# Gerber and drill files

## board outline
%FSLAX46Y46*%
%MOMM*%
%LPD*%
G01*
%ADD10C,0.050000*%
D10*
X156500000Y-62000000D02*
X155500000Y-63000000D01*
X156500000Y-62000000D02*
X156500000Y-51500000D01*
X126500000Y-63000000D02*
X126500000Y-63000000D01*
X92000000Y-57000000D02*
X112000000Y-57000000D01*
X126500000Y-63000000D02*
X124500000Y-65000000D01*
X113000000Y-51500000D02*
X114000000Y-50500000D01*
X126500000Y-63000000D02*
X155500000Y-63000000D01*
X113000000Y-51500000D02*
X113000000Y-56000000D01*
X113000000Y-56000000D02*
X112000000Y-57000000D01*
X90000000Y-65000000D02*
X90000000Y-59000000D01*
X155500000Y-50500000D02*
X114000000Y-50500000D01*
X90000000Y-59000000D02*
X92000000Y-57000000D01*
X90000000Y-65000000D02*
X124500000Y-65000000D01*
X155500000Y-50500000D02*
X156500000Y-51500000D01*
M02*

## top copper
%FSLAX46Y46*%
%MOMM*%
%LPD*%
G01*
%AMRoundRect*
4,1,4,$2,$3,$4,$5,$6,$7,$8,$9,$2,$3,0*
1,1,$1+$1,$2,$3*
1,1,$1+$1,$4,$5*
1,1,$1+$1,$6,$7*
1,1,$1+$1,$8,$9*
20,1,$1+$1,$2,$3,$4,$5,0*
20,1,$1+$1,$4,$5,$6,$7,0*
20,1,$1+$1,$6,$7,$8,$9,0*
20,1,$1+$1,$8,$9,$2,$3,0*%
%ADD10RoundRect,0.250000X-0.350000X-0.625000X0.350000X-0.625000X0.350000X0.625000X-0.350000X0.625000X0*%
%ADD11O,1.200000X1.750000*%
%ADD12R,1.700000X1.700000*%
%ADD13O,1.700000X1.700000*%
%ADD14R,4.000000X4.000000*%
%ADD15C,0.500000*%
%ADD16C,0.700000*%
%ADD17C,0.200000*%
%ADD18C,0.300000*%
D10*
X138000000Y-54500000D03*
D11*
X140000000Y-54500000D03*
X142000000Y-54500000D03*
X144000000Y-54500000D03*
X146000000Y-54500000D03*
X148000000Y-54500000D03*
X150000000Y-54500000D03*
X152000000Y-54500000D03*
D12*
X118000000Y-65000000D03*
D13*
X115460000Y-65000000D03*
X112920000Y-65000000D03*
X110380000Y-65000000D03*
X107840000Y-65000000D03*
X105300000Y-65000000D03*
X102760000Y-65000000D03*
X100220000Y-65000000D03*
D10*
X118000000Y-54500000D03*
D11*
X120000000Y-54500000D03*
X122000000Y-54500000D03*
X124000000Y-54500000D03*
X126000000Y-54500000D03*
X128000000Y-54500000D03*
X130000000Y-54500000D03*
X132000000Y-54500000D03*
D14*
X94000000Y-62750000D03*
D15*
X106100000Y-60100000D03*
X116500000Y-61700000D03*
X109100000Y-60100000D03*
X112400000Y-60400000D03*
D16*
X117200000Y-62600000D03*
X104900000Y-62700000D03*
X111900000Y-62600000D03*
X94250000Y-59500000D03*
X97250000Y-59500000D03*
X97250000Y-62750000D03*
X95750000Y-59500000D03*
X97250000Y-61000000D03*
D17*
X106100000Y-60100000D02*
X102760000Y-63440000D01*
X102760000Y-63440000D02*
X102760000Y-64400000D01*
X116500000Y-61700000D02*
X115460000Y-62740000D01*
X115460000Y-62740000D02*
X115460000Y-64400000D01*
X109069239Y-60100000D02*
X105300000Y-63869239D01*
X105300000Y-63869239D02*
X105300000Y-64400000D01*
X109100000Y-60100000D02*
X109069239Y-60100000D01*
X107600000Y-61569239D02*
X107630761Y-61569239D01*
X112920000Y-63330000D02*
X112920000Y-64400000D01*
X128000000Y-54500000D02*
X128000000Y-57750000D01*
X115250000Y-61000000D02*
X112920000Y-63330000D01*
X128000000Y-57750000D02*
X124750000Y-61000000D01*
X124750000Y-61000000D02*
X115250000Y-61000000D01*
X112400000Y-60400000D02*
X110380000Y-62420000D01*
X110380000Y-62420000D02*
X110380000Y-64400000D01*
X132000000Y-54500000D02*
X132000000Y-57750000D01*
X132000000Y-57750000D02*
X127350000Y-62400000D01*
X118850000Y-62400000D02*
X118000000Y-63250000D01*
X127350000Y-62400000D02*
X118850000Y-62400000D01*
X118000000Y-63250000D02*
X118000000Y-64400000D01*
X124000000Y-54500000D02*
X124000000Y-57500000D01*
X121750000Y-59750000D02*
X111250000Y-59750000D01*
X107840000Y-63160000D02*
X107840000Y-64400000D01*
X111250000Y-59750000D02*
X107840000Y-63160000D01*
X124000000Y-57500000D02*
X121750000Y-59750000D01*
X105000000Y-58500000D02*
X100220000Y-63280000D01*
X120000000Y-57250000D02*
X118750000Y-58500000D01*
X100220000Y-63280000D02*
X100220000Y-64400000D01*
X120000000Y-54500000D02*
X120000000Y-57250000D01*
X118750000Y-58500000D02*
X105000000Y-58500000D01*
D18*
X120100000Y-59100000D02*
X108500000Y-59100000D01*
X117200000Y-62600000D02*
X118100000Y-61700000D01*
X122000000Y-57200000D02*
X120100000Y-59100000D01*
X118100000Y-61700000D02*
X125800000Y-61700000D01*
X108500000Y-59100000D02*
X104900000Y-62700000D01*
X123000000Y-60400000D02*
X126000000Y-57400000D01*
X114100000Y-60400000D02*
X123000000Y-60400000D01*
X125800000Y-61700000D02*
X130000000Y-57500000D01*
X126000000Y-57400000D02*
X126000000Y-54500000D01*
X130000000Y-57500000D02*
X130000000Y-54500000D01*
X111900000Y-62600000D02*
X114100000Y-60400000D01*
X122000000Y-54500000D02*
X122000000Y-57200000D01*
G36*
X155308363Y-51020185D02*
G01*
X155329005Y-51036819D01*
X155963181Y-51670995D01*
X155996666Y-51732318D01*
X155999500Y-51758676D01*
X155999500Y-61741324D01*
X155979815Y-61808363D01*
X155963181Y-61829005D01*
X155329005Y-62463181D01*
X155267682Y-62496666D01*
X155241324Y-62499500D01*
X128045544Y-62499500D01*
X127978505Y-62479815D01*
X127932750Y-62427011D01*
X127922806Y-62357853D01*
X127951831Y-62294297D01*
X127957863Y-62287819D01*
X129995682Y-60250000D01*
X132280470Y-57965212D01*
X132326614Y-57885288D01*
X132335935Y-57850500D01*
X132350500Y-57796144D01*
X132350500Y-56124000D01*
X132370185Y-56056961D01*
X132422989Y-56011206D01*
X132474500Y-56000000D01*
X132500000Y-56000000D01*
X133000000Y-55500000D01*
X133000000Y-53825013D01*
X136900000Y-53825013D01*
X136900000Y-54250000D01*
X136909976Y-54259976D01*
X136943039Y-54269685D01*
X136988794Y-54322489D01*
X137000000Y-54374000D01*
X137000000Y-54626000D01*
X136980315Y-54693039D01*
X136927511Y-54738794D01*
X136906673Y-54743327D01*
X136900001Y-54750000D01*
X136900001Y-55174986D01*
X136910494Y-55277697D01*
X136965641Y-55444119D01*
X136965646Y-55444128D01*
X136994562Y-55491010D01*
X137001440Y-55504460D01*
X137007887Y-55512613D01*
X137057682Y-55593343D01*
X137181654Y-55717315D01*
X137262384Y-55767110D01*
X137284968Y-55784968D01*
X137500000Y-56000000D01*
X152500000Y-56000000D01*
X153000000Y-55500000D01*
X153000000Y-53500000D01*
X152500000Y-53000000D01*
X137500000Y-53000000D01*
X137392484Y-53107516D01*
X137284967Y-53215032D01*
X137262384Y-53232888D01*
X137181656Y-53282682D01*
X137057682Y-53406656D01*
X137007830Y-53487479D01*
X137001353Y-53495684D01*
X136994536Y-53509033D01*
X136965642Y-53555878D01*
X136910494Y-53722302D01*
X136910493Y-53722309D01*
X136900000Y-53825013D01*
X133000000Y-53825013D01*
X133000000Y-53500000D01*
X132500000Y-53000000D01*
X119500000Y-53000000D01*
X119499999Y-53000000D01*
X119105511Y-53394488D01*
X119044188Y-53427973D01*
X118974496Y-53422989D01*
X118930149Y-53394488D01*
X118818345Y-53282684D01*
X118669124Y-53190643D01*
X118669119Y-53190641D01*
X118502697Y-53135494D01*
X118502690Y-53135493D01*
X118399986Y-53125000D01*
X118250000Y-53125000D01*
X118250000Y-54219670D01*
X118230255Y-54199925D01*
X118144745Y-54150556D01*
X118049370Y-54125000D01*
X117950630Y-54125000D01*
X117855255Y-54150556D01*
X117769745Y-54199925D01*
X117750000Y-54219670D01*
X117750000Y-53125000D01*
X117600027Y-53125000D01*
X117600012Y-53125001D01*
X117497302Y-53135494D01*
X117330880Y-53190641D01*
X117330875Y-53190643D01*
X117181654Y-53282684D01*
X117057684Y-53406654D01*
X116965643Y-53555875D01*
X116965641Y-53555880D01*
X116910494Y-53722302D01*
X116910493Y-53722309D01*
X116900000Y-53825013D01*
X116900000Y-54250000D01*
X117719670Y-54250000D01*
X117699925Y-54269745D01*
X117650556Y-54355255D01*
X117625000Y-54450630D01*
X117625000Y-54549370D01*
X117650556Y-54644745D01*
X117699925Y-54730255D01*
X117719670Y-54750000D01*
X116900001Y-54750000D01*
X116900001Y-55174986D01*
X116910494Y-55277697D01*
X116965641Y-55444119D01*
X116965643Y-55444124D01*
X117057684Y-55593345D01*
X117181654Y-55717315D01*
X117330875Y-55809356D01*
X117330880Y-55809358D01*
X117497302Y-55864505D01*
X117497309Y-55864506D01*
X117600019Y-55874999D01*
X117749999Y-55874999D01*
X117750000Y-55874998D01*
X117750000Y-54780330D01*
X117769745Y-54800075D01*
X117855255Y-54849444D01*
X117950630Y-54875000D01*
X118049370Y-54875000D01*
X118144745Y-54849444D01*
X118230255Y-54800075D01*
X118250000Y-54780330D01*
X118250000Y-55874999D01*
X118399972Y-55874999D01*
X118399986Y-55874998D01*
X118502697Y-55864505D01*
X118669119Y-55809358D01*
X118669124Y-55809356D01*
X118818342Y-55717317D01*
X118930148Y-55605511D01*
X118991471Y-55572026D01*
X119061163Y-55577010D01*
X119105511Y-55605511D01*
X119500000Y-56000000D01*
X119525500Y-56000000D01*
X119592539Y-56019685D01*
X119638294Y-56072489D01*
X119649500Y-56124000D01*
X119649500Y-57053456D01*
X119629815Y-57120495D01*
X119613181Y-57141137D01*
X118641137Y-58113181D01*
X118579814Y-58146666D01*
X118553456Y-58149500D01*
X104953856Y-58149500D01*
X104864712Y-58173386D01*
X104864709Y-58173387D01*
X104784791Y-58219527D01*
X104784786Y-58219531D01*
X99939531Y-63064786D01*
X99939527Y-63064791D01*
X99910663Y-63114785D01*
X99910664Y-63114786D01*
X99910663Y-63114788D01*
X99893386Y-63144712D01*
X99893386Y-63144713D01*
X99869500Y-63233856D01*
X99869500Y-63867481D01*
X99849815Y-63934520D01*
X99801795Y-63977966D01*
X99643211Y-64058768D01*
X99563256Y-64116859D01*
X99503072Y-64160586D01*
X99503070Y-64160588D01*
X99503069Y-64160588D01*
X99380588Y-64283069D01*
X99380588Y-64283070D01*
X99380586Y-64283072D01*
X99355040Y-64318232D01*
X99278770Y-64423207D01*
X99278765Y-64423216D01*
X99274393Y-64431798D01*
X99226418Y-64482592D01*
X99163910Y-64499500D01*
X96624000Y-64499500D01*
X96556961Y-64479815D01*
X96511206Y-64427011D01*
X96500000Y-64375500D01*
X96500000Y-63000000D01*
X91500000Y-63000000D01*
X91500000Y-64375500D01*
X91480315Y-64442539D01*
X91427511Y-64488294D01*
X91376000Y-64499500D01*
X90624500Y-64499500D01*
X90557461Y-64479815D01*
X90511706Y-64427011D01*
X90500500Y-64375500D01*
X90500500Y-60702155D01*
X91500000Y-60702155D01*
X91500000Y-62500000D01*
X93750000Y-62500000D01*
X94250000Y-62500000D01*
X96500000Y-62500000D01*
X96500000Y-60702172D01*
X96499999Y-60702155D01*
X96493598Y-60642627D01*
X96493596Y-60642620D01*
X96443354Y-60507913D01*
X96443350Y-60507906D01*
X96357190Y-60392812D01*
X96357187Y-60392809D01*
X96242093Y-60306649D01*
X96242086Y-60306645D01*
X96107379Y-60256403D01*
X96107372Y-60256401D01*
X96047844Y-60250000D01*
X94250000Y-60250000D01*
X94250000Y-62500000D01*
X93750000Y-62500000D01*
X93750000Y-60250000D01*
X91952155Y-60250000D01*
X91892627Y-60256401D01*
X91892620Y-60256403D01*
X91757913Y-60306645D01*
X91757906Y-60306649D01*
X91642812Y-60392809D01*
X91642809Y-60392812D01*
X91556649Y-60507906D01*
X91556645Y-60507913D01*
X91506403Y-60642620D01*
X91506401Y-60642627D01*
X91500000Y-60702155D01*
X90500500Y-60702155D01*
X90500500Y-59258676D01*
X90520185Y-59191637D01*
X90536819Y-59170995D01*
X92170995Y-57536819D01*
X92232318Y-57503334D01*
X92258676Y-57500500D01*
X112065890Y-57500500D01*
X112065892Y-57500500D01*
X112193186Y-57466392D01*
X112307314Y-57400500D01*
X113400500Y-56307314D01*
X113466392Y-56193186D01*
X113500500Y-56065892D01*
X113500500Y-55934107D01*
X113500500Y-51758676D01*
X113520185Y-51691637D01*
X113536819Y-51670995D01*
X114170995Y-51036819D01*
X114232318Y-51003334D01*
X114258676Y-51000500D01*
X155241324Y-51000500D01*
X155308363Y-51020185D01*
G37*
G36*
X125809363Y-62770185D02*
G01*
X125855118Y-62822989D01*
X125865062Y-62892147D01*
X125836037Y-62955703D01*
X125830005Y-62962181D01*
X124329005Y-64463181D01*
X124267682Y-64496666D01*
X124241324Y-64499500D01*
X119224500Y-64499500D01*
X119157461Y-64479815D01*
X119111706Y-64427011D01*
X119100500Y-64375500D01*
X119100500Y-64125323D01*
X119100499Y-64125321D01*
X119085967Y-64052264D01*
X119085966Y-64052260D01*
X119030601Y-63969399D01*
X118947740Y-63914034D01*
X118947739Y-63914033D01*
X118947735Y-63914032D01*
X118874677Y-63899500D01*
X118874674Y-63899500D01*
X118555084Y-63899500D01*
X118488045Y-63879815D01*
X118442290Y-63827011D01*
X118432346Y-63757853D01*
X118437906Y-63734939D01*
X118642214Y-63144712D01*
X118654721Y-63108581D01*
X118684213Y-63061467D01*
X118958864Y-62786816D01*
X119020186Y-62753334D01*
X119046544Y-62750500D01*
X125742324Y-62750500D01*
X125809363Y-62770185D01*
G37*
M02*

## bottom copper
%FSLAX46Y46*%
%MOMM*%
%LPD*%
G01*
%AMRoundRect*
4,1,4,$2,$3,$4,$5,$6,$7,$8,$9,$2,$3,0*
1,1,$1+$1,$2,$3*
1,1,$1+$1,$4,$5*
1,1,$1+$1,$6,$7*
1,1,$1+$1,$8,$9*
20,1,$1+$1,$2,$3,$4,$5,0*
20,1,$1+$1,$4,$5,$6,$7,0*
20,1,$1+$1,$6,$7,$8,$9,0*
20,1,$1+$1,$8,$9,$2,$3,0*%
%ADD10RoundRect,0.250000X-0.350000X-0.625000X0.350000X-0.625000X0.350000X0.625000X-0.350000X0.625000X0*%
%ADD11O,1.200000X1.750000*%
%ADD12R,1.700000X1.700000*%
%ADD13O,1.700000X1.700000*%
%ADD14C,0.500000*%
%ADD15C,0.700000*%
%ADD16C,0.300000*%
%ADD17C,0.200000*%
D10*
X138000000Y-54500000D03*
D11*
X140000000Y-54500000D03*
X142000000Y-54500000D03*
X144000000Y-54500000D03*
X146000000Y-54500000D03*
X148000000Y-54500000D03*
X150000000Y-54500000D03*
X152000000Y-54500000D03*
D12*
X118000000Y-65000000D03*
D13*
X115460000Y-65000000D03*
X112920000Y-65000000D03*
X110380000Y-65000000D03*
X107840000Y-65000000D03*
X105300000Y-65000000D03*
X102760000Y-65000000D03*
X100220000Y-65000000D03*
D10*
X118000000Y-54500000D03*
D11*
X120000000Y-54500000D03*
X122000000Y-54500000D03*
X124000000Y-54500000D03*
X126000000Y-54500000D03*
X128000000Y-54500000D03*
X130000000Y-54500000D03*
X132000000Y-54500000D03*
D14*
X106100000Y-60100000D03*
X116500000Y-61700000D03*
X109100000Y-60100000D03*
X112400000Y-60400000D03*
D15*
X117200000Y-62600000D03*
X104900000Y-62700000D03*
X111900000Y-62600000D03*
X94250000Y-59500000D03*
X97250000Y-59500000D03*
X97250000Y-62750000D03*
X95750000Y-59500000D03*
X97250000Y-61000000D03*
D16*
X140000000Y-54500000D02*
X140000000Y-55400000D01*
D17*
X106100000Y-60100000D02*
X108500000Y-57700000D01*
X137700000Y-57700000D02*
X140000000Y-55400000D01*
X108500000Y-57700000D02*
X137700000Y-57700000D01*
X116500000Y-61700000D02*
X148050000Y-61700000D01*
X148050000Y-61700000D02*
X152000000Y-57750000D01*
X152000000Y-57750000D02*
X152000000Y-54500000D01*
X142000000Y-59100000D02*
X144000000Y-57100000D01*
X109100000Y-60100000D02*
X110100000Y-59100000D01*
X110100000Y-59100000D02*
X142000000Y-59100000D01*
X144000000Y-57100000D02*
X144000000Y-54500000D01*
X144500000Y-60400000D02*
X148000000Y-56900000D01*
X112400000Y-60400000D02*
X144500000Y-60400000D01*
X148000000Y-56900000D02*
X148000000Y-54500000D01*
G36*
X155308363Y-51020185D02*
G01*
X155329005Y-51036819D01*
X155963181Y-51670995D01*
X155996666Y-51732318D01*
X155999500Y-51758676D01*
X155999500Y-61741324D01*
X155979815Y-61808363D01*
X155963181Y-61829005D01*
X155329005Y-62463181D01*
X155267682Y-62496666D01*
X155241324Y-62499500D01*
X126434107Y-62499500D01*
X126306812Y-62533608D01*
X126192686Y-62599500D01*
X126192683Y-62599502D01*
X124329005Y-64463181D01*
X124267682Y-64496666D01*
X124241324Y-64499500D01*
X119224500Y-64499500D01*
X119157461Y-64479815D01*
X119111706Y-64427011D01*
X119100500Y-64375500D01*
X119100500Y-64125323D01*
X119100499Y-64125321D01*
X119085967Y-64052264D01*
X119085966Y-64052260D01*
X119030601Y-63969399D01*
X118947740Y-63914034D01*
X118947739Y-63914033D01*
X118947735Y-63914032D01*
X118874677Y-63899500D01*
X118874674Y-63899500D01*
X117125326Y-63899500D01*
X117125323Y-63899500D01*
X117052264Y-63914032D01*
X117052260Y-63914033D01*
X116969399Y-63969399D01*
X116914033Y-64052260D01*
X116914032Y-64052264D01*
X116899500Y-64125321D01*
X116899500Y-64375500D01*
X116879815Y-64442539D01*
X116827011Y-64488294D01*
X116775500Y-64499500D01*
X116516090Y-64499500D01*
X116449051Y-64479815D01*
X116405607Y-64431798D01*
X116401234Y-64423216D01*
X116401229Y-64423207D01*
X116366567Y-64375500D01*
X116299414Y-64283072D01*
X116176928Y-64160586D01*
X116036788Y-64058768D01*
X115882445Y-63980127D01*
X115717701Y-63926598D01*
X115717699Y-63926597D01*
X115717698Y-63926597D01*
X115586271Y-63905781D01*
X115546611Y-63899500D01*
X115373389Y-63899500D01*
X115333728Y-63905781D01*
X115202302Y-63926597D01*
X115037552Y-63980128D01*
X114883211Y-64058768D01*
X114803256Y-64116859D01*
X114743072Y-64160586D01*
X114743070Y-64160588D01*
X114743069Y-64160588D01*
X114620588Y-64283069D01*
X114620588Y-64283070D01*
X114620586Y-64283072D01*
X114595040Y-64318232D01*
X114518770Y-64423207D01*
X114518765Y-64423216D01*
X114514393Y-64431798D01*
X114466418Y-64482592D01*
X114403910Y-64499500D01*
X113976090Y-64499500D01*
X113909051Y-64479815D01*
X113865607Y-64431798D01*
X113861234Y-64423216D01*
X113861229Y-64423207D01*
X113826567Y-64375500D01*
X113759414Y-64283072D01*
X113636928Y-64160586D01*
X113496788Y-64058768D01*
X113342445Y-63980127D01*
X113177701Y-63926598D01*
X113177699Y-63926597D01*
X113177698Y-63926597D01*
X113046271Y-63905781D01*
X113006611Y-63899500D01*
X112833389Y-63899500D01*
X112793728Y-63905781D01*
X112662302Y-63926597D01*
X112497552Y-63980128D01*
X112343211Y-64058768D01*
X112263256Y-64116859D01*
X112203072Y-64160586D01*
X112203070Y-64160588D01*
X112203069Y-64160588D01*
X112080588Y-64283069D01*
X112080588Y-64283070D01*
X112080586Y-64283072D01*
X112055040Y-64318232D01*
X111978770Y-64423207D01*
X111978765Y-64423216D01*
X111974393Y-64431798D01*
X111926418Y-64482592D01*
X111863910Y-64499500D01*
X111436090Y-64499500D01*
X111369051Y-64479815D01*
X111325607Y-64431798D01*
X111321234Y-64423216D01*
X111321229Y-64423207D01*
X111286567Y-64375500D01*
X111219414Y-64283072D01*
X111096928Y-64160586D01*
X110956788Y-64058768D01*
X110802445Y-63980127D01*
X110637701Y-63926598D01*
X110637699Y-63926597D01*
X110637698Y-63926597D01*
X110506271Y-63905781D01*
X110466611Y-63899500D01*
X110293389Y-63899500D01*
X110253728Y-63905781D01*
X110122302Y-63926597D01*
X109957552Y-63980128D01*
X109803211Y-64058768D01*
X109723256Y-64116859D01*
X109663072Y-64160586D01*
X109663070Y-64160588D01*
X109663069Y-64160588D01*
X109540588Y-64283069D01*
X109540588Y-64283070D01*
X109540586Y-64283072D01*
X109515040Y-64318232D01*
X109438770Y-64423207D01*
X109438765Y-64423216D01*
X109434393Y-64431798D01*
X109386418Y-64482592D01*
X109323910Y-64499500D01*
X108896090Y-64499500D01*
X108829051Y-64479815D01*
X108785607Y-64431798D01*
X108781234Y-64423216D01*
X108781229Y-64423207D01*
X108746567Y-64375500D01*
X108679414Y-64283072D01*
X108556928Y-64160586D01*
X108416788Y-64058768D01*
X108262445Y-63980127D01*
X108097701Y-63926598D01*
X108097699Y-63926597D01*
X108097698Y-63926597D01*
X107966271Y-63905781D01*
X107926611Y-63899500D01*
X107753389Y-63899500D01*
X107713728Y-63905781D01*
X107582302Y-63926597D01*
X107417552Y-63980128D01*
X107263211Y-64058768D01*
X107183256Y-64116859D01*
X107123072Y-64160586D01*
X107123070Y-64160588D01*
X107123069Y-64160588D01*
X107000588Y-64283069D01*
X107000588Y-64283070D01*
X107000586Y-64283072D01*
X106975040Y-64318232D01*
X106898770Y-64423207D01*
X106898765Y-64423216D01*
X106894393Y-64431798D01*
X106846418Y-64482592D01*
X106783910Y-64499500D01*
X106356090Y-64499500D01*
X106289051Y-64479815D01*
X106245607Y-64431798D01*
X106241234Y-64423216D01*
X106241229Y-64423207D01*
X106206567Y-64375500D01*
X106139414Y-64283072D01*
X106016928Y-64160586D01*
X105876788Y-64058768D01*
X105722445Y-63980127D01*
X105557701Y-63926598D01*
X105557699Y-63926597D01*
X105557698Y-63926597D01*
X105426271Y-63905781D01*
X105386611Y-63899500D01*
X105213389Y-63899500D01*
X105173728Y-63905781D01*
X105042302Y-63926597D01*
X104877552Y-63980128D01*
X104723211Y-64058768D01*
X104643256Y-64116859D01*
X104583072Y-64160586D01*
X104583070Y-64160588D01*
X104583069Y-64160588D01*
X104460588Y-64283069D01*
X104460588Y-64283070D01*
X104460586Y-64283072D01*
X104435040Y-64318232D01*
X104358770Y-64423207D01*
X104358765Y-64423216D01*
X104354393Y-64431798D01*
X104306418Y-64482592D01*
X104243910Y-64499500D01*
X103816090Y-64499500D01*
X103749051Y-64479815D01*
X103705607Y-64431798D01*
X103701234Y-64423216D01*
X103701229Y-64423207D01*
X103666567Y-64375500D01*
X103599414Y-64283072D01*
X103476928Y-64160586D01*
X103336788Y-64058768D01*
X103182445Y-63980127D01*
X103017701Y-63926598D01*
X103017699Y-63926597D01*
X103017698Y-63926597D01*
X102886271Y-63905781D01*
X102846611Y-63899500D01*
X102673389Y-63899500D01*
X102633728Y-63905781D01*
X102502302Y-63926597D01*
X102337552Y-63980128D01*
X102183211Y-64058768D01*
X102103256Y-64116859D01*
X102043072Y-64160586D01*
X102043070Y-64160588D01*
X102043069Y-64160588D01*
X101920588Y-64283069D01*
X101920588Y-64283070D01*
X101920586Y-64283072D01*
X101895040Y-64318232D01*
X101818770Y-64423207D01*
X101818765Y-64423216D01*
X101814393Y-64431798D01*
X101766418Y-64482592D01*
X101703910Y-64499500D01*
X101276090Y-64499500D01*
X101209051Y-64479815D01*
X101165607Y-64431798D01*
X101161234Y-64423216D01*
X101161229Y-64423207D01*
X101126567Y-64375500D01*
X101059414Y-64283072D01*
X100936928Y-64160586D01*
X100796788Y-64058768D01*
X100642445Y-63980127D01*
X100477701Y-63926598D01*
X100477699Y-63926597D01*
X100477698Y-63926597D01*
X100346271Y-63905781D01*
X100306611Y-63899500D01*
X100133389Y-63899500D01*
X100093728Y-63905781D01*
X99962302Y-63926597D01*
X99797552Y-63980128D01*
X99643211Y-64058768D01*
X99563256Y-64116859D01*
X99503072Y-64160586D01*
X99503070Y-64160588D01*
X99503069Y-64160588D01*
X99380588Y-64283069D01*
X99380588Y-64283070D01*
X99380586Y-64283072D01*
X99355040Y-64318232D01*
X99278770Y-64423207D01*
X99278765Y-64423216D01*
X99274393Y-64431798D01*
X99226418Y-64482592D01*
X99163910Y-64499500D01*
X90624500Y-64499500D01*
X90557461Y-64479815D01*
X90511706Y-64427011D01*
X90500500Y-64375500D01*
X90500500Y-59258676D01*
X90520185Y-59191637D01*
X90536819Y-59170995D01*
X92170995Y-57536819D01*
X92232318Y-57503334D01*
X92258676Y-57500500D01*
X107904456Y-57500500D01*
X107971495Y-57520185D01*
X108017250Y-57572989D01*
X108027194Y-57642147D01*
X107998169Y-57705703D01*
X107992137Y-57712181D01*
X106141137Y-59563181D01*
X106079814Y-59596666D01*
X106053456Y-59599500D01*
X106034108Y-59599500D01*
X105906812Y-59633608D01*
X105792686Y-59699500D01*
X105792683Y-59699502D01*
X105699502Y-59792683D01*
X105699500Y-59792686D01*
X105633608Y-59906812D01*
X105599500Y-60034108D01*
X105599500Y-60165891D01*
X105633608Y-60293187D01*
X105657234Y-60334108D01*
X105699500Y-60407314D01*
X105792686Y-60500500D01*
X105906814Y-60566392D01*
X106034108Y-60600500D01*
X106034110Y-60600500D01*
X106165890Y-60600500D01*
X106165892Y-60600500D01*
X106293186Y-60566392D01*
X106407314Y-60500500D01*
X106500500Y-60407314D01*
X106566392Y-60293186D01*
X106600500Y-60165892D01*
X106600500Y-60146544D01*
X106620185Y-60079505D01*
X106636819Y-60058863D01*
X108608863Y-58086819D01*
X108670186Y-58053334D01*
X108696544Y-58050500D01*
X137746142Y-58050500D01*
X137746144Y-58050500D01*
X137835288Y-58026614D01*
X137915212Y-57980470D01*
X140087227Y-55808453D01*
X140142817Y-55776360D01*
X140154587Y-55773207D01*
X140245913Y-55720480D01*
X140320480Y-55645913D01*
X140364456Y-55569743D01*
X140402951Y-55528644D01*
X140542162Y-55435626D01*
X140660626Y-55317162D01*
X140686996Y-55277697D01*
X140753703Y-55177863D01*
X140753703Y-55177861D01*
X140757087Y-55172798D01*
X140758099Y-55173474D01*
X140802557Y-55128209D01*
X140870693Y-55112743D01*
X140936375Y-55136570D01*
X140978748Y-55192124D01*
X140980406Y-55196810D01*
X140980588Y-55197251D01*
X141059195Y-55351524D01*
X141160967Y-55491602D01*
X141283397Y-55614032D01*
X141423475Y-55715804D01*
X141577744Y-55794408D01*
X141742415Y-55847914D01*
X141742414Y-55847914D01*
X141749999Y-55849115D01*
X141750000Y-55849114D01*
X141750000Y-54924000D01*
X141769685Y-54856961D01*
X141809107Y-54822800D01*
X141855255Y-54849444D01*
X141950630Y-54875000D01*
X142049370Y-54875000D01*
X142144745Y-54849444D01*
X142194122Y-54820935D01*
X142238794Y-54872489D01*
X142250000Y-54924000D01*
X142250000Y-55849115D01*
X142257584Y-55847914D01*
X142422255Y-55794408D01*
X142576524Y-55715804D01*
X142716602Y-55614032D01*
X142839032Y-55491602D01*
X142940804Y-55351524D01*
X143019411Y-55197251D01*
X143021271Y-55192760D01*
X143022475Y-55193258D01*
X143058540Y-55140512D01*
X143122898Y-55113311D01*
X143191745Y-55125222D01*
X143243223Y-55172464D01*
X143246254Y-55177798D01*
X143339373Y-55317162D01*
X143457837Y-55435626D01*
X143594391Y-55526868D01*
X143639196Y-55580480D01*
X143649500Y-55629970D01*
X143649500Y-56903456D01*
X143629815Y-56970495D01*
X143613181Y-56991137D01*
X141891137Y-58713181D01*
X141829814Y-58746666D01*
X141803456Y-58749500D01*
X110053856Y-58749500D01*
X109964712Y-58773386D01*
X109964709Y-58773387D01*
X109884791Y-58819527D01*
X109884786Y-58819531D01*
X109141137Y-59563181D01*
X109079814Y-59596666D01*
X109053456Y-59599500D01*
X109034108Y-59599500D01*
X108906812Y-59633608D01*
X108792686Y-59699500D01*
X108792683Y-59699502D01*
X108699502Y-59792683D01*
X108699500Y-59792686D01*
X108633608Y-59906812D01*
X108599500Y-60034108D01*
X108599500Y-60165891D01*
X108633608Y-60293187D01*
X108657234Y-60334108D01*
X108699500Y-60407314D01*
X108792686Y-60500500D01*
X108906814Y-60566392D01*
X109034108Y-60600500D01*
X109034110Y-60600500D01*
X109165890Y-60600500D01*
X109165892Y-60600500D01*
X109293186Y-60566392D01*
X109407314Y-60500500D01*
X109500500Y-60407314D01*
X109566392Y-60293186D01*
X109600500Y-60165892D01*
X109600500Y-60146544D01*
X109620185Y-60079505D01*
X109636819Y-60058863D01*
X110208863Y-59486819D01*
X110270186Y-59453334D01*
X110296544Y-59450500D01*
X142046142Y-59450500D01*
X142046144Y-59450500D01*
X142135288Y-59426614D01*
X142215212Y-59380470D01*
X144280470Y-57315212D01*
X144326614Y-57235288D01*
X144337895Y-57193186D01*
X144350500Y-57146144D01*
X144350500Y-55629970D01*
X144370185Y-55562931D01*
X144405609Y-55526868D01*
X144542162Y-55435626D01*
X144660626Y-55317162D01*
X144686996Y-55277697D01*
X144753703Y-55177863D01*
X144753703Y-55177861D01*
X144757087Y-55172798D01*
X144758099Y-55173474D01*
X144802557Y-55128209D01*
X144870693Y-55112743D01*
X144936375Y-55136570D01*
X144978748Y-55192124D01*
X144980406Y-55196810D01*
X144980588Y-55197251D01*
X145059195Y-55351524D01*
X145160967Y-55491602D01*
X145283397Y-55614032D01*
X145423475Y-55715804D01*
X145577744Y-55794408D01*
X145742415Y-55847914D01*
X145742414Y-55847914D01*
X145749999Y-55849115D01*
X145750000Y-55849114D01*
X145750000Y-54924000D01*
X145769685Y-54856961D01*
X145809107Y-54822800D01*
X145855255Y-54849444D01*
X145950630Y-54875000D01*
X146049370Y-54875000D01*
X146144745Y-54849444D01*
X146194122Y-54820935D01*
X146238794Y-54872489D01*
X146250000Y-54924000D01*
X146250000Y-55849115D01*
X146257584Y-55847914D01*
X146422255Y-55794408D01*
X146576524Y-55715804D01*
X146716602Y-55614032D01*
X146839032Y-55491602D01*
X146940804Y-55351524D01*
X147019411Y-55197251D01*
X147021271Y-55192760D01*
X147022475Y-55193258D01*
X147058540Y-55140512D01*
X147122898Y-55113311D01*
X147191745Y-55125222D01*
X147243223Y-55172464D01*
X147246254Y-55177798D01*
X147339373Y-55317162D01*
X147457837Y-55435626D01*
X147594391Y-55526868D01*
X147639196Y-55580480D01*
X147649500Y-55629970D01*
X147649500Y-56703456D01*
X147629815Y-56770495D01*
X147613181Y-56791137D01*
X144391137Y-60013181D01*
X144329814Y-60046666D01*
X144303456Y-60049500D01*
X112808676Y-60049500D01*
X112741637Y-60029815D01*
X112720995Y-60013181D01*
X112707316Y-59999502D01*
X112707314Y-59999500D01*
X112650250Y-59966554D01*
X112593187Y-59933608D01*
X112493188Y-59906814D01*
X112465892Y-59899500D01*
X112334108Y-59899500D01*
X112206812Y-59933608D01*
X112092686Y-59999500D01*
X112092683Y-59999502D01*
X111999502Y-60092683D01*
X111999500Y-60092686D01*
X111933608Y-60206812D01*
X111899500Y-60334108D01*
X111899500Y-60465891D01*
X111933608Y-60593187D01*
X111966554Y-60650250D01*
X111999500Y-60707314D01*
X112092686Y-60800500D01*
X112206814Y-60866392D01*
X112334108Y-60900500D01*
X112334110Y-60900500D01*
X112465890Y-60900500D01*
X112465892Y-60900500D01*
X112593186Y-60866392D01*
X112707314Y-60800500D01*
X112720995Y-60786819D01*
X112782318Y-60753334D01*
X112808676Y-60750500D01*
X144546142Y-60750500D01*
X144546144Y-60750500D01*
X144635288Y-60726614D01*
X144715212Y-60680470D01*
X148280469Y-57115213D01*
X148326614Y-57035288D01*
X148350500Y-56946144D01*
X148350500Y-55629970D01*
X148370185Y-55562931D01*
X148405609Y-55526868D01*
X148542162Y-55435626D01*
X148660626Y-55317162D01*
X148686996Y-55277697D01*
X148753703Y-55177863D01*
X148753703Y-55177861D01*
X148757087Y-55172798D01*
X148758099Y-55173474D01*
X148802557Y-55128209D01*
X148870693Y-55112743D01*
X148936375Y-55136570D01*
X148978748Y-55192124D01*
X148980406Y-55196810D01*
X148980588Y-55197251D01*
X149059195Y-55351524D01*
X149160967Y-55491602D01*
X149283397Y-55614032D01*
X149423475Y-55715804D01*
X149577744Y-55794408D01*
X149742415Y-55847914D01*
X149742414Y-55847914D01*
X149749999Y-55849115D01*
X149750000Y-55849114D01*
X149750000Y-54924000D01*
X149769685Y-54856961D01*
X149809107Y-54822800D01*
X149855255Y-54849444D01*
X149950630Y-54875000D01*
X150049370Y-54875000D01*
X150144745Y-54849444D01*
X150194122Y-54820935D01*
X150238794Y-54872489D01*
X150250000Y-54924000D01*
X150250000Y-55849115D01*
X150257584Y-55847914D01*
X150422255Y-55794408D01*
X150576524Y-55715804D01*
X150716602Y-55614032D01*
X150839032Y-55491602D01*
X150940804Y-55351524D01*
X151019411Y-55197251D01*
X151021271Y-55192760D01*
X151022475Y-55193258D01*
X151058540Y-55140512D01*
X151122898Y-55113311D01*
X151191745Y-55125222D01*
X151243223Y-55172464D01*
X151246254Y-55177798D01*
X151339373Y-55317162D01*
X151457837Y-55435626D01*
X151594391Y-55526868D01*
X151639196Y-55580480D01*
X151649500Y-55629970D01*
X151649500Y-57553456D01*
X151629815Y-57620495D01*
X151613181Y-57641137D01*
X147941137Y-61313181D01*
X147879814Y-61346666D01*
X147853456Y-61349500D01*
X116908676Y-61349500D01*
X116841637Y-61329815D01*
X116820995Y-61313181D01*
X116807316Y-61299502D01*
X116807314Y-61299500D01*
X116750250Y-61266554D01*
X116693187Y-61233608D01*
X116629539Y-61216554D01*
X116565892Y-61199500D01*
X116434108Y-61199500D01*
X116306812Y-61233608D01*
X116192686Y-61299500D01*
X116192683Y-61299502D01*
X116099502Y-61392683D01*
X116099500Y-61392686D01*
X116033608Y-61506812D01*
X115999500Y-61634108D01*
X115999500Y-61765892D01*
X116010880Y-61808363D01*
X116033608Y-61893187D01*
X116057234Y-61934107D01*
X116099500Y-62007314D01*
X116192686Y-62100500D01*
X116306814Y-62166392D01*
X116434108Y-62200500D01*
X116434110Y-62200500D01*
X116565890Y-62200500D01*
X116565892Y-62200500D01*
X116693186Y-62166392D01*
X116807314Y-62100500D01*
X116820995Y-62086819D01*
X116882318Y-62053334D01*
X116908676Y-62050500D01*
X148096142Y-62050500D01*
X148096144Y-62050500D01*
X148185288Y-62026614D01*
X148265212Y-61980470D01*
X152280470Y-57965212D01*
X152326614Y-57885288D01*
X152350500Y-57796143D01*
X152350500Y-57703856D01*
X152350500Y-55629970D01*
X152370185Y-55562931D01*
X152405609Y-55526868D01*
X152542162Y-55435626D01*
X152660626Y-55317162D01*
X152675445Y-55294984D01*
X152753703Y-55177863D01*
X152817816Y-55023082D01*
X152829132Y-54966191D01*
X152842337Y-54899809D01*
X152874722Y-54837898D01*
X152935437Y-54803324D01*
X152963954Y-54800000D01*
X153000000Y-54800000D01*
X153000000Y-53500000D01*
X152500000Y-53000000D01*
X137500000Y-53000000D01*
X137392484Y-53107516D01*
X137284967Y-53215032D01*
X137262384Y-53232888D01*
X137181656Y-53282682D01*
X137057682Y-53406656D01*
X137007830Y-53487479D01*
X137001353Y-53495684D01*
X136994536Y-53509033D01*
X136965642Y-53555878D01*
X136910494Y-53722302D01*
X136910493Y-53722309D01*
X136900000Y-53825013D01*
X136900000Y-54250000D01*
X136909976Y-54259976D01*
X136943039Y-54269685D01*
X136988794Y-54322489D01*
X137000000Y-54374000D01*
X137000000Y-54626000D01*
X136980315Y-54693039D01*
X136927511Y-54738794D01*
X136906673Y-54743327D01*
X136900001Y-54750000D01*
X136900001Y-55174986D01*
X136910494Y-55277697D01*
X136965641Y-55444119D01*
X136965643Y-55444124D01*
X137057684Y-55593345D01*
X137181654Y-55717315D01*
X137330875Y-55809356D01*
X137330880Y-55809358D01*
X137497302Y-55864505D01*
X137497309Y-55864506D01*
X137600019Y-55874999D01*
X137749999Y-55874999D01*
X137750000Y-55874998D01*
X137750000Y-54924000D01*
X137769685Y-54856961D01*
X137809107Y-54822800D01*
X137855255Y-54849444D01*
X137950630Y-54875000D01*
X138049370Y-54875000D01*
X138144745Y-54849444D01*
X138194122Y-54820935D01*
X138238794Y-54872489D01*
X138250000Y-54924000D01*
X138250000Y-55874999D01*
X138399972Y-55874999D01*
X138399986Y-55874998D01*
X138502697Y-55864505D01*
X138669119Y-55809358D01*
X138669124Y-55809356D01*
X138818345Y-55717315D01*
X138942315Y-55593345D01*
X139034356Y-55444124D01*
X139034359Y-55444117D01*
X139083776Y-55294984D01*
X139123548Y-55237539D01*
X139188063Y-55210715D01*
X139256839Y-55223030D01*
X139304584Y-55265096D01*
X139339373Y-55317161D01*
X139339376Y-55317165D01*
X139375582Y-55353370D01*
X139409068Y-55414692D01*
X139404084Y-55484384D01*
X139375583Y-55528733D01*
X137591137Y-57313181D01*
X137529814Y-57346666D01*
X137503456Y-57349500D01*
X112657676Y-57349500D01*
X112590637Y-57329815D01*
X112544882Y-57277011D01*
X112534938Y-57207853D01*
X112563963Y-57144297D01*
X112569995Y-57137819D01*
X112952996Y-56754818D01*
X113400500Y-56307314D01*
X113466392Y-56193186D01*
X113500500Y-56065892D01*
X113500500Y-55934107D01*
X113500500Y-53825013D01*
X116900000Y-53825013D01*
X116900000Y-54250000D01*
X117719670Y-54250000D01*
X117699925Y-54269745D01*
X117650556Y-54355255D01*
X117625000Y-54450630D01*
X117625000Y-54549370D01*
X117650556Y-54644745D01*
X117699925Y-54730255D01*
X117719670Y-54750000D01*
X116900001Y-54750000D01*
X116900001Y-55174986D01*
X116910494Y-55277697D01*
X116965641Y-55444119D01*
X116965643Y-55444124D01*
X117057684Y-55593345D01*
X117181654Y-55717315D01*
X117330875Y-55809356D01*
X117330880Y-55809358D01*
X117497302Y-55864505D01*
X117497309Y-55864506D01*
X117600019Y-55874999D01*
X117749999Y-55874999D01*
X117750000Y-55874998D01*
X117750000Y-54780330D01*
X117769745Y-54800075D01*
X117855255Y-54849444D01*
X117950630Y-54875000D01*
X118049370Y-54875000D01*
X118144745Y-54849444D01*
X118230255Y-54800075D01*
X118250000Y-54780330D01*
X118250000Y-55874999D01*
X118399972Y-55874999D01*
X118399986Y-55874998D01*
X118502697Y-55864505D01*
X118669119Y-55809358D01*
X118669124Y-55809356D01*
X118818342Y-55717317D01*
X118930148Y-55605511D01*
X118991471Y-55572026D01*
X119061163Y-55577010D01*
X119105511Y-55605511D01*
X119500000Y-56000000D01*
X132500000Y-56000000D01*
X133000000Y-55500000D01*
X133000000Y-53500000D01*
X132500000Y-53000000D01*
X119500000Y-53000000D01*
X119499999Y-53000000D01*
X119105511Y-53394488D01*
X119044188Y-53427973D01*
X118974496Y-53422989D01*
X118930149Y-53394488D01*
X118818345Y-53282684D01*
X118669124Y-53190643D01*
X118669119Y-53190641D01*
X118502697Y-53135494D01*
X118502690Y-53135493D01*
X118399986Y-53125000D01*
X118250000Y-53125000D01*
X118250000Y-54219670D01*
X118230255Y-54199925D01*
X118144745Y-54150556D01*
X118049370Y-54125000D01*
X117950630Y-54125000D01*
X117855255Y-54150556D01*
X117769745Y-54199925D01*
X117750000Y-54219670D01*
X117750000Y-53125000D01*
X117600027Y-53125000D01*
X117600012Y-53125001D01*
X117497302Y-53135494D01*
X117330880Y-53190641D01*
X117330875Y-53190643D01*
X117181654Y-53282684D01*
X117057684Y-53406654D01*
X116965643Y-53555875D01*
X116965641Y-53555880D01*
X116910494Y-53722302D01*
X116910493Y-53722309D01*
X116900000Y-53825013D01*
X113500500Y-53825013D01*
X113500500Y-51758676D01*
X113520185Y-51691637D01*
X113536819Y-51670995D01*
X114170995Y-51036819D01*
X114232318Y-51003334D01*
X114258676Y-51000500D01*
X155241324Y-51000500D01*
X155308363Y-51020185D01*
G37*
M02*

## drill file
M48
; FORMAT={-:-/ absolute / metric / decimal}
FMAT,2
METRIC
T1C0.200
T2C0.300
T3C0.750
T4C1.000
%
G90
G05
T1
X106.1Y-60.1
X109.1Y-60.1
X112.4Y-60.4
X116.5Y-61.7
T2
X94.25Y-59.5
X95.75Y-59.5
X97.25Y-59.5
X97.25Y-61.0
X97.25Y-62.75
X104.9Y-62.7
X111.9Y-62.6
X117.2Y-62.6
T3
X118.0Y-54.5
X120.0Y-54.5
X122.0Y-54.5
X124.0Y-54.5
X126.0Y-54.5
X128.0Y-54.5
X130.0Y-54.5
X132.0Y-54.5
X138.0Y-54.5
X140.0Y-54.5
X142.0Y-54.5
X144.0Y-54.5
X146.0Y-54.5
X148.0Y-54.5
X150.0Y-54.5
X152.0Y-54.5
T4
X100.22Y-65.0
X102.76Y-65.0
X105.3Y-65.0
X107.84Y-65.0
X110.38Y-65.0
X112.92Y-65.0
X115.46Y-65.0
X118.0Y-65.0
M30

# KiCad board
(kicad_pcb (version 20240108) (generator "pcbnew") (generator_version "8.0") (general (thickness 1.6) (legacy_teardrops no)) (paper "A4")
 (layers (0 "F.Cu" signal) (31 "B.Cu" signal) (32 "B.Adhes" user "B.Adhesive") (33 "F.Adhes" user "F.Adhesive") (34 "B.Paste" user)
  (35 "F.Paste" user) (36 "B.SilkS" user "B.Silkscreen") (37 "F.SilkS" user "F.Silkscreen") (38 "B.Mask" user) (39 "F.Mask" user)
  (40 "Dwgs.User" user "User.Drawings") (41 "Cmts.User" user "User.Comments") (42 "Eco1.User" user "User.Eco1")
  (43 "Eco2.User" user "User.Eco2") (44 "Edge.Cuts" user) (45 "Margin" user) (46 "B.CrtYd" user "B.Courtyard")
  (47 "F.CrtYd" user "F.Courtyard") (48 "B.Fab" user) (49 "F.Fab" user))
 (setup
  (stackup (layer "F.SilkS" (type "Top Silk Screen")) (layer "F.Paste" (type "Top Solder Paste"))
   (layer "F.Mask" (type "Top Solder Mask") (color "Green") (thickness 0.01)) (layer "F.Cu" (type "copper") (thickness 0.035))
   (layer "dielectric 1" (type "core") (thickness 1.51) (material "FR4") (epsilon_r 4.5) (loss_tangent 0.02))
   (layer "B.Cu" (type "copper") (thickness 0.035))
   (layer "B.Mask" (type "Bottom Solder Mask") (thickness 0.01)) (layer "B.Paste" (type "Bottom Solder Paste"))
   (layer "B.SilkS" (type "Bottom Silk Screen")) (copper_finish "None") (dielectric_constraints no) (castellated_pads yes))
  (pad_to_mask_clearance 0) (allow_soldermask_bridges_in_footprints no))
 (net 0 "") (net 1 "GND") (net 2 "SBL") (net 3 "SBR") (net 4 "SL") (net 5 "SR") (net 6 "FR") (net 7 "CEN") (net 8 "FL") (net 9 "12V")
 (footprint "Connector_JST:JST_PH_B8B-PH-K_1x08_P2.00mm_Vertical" (layer "F.Cu") (at 138 54.5)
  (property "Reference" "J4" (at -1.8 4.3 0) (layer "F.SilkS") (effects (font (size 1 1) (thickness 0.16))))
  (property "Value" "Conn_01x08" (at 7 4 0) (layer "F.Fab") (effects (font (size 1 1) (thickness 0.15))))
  (pad "1" thru_hole roundrect (at 0 0) (size 1.2 1.75) (drill 0.75) (layers "*.Cu" "*.Mask") (remove_unused_layers no)
   (roundrect_rratio 0.208333) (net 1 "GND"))
  (pad "2" thru_hole oval (at 2 0) (size 1.2 1.75) (drill 0.75) (layers "*.Cu" "*.Mask") (remove_unused_layers no) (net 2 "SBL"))
  (pad "3" thru_hole oval (at 4 0) (size 1.2 1.75) (drill 0.75) (layers "*.Cu" "*.Mask") (remove_unused_layers no) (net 1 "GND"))
  (pad "4" thru_hole oval (at 6 0) (size 1.2 1.75) (drill 0.75) (layers "*.Cu" "*.Mask") (remove_unused_layers no) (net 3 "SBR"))
  (pad "5" thru_hole oval (at 8 0) (size 1.2 1.75) (drill 0.75) (layers "*.Cu" "*.Mask") (remove_unused_layers no) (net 1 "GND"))
  (pad "6" thru_hole oval (at 10 0) (size 1.2 1.75) (drill 0.75) (layers "*.Cu" "*.Mask") (remove_unused_layers no) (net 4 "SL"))
  (pad "7" thru_hole oval (at 12 0) (size 1.2 1.75) (drill 0.75) (layers "*.Cu" "*.Mask") (remove_unused_layers no) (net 1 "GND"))
  (pad "8" thru_hole oval (at 14 0) (size 1.2 1.75) (drill 0.75) (layers "*.Cu" "*.Mask") (remove_unused_layers no) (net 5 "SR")))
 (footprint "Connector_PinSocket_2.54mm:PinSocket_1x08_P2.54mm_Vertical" (layer "F.Cu") (at 118 65 -90)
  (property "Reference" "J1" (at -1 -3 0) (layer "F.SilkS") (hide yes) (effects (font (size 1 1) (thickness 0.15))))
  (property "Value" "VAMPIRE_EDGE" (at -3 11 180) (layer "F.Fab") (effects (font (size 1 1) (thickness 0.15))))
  (pad "1" thru_hole rect (at 0 0 270) (size 1.7 1.7) (drill 1) (layers "*.Cu" "*.Mask") (remove_unused_layers no) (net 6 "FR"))
  (pad "2" thru_hole oval (at 0 2.54 270) (size 1.7 1.7) (drill 1) (layers "*.Cu" "*.Mask") (remove_unused_layers no) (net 5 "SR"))
  (pad "3" thru_hole oval (at 0 5.08 270) (size 1.7 1.7) (drill 1) (layers "*.Cu" "*.Mask") (remove_unused_layers no) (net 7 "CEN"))
  (pad "4" thru_hole oval (at 0 7.62 270) (size 1.7 1.7) (drill 1) (layers "*.Cu" "*.Mask") (remove_unused_layers no) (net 4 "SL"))
  (pad "5" thru_hole oval (at 0 10.16 270) (size 1.7 1.7) (drill 1) (layers "*.Cu" "*.Mask") (remove_unused_layers no) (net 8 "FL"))
  (pad "6" thru_hole oval (at 0 12.7 270) (size 1.7 1.7) (drill 1) (layers "*.Cu" "*.Mask") (remove_unused_layers no) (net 3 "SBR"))
  (pad "7" thru_hole oval (at 0 15.24 270) (size 1.7 1.7) (drill 1) (layers "*.Cu" "*.Mask") (remove_unused_layers no) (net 2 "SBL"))
  (pad "8" thru_hole oval (at 0 17.78 270) (size 1.7 1.7) (drill 1) (layers "*.Cu" "*.Mask") (remove_unused_layers no) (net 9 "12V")))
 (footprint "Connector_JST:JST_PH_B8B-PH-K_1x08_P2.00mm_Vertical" (layer "F.Cu") (at 118 54.5)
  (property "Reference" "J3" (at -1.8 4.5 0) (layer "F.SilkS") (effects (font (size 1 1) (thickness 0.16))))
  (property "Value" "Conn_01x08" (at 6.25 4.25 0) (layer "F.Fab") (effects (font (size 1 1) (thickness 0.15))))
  (pad "1" thru_hole roundrect (at 0 0) (size 1.2 1.75) (drill 0.75) (layers "*.Cu" "*.Mask") (remove_unused_layers no)
   (roundrect_rratio 0.208333) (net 1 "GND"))
  (pad "2" thru_hole oval (at 2 0) (size 1.2 1.75) (drill 0.75) (layers "*.Cu" "*.Mask") (remove_unused_layers no) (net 9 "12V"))
  (pad "3" thru_hole oval (at 4 0) (size 1.2 1.75) (drill 0.75) (layers "*.Cu" "*.Mask") (remove_unused_layers no) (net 1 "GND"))
  (pad "4" thru_hole oval (at 6 0) (size 1.2 1.75) (drill 0.75) (layers "*.Cu" "*.Mask") (remove_unused_layers no) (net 8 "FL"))
  (pad "5" thru_hole oval (at 8 0) (size 1.2 1.75) (drill 0.75) (layers "*.Cu" "*.Mask") (remove_unused_layers no) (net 1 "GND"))
  (pad "6" thru_hole oval (at 10 0) (size 1.2 1.75) (drill 0.75) (layers "*.Cu" "*.Mask") (remove_unused_layers no) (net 7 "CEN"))
  (pad "7" thru_hole oval (at 12 0) (size 1.2 1.75) (drill 0.75) (layers "*.Cu" "*.Mask") (remove_unused_layers no) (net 1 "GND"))
  (pad "8" thru_hole oval (at 14 0) (size 1.2 1.75) (drill 0.75) (layers "*.Cu" "*.Mask") (remove_unused_layers no) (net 6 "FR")))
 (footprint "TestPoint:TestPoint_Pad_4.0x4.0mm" (layer "F.Cu") (at 94 62.75 90)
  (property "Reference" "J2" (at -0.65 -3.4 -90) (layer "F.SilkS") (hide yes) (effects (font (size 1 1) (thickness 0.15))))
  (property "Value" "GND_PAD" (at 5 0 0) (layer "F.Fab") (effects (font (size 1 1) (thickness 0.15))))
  (pad "1" smd rect (at 0 0 90) (size 4 4) (layers "F.Cu" "F.Mask") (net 1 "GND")))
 (gr_line (start 156.5 62) (end 155.5 63) (stroke (width 0.05) (type default)) (layer "Edge.Cuts"))
 (gr_line (start 156.5 62) (end 156.5 51.5) (stroke (width 0.05) (type default)) (layer "Edge.Cuts"))
 (gr_line (start 126.5 63) (end 126.5 63) (stroke (width 0.05) (type default)) (layer "Edge.Cuts"))
 (gr_line (start 92 57) (end 112 57) (stroke (width 0.05) (type default)) (layer "Edge.Cuts"))
 (gr_line (start 126.5 63) (end 124.5 65) (stroke (width 0.05) (type default)) (layer "Edge.Cuts"))
 (gr_line (start 113 51.5) (end 114 50.5) (stroke (width 0.05) (type default)) (layer "Edge.Cuts"))
 (gr_line (start 126.5 63) (end 155.5 63) (stroke (width 0.05) (type default)) (layer "Edge.Cuts"))
 (gr_line (start 113 51.5) (end 113 56) (stroke (width 0.05) (type default)) (layer "Edge.Cuts"))
 (gr_line (start 113 56) (end 112 57) (stroke (width 0.05) (type default)) (layer "Edge.Cuts"))
 (gr_line (start 90 65) (end 90 59) (stroke (width 0.05) (type default)) (layer "Edge.Cuts"))
 (gr_line (start 155.5 50.5) (end 114 50.5) (stroke (width 0.05) (type default)) (layer "Edge.Cuts"))
 (gr_line (start 90 59) (end 92 57) (stroke (width 0.05) (type default)) (layer "Edge.Cuts"))
 (gr_line (start 90 65) (end 124.5 65) (stroke (width 0.05) (type default)) (layer "Edge.Cuts"))
 (gr_line (start 155.5 50.5) (end 156.5 51.5) (stroke (width 0.05) (type default)) (layer "Edge.Cuts"))
 (segment (start 106.1 60.1) (end 102.76 63.44) (width 0.2) (layer "F.Cu") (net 2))
 (segment (start 102.76 63.44) (end 102.76 64.4) (width 0.2) (layer "F.Cu") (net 2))
 (via (at 106.1 60.1) (size 0.5) (drill 0.2) (layers "F.Cu" "B.Cu") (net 2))
 (segment (start 140 54.5) (end 140 55.4) (width 0.3) (layer "B.Cu") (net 2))
 (segment (start 106.1 60.1) (end 108.5 57.7) (width 0.2) (layer "B.Cu") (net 2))
 (segment (start 137.7 57.7) (end 140 55.4) (width 0.2) (layer "B.Cu") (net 2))
 (segment (start 108.5 57.7) (end 137.7 57.7) (width 0.2) (layer "B.Cu") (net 2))
 (segment (start 116.5 61.7) (end 115.46 62.74) (width 0.2) (layer "F.Cu") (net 5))
 (segment (start 115.46 62.74) (end 115.46 64.4) (width 0.2) (layer "F.Cu") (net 5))
 (via (at 116.5 61.7) (size 0.5) (drill 0.2) (layers "F.Cu" "B.Cu") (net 5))
 (segment (start 116.5 61.7) (end 148.05 61.7) (width 0.2) (layer "B.Cu") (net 5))
 (segment (start 148.05 61.7) (end 152 57.75) (width 0.2) (layer "B.Cu") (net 5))
 (segment (start 152 57.75) (end 152 54.5) (width 0.2) (layer "B.Cu") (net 5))
 (segment (start 109.069239 60.1) (end 105.3 63.869239) (width 0.2) (layer "F.Cu") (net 3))
 (segment (start 105.3 63.869239) (end 105.3 64.4) (width 0.2) (layer "F.Cu") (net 3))
 (segment (start 109.1 60.1) (end 109.069239 60.1) (width 0.2) (layer "F.Cu") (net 3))
 (segment (start 107.6 61.569239) (end 107.630761 61.569239) (width 0.2) (layer "F.Cu") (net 3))
 (via (at 109.1 60.1) (size 0.5) (drill 0.2) (layers "F.Cu" "B.Cu") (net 3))
 (segment (start 142 59.1) (end 144 57.1) (width 0.2) (layer "B.Cu") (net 3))
 (segment (start 109.1 60.1) (end 110.1 59.1) (width 0.2) (layer "B.Cu") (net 3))
 (segment (start 110.1 59.1) (end 142 59.1) (width 0.2) (layer "B.Cu") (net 3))
 (segment (start 144 57.1) (end 144 54.5) (width 0.2) (layer "B.Cu") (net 3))
 (segment (start 112.92 63.33) (end 112.92 64.4) (width 0.2) (layer "F.Cu") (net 7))
 (segment (start 128 54.5) (end 128 57.75) (width 0.2) (layer "F.Cu") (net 7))
 (segment (start 115.25 61) (end 112.92 63.33) (width 0.2) (layer "F.Cu") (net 7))
 (segment (start 128 57.75) (end 124.75 61) (width 0.2) (layer "F.Cu") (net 7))
 (segment (start 124.75 61) (end 115.25 61) (width 0.2) (layer "F.Cu") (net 7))
 (segment (start 112.4 60.4) (end 110.38 62.42) (width 0.2) (layer "F.Cu") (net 4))
 (segment (start 110.38 62.42) (end 110.38 64.4) (width 0.2) (layer "F.Cu") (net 4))
 (via (at 112.4 60.4) (size 0.5) (drill 0.2) (layers "F.Cu" "B.Cu") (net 4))
 (segment (start 144.5 60.4) (end 148 56.9) (width 0.2) (layer "B.Cu") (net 4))
 (segment (start 112.4 60.4) (end 144.5 60.4) (width 0.2) (layer "B.Cu") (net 4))
 (segment (start 148 56.9) (end 148 54.5) (width 0.2) (layer "B.Cu") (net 4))
 (segment (start 132 54.5) (end 132 57.75) (width 0.2) (layer "F.Cu") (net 6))
 (segment (start 132 57.75) (end 127.35 62.4) (width 0.2) (layer "F.Cu") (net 6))
 (segment (start 118.85 62.4) (end 118 63.25) (width 0.2) (layer "F.Cu") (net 6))
 (segment (start 127.35 62.4) (end 118.85 62.4) (width 0.2) (layer "F.Cu") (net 6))
 (segment (start 118 63.25) (end 118 64.4) (width 0.2) (layer "F.Cu") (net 6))
 (segment (start 124 54.5) (end 124 57.5) (width 0.2) (layer "F.Cu") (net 8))
 (segment (start 121.75 59.75) (end 111.25 59.75) (width 0.2) (layer "F.Cu") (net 8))
 (segment (start 107.84 63.16) (end 107.84 64.4) (width 0.2) (layer "F.Cu") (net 8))
 (segment (start 111.25 59.75) (end 107.84 63.16) (width 0.2) (layer "F.Cu") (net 8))
 (segment (start 124 57.5) (end 121.75 59.75) (width 0.2) (layer "F.Cu") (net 8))
 (segment (start 105 58.5) (end 100.22 63.28) (width 0.2) (layer "F.Cu") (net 9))
 (segment (start 120 57.25) (end 118.75 58.5) (width 0.2) (layer "F.Cu") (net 9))
 (segment (start 100.22 63.28) (end 100.22 64.4) (width 0.2) (layer "F.Cu") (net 9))
 (segment (start 120 54.5) (end 120 57.25) (width 0.2) (layer "F.Cu") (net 9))
 (segment (start 118.75 58.5) (end 105 58.5) (width 0.2) (layer "F.Cu") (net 9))
 (segment (start 120.1 59.1) (end 108.5 59.1) (width 0.3) (layer "F.Cu") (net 1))
 (segment (start 117.2 62.6) (end 118.1 61.7) (width 0.3) (layer "F.Cu") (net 1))
 (segment (start 122 57.2) (end 120.1 59.1) (width 0.3) (layer "F.Cu") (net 1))
 (segment (start 118.1 61.7) (end 125.8 61.7) (width 0.3) (layer "F.Cu") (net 1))
 (segment (start 108.5 59.1) (end 104.9 62.7) (width 0.3) (layer "F.Cu") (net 1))
 (segment (start 123 60.4) (end 126 57.4) (width 0.3) (layer "F.Cu") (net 1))
 (segment (start 114.1 60.4) (end 123 60.4) (width 0.3) (layer "F.Cu") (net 1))
 (segment (start 125.8 61.7) (end 130 57.5) (width 0.3) (layer "F.Cu") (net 1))
 (segment (start 126 57.4) (end 126 54.5) (width 0.3) (layer "F.Cu") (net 1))
 (segment (start 130 57.5) (end 130 54.5) (width 0.3) (layer "F.Cu") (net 1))
 (segment (start 111.9 62.6) (end 114.1 60.4) (width 0.3) (layer "F.Cu") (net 1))
 (segment (start 122 54.5) (end 122 57.2) (width 0.3) (layer "F.Cu") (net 1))
 (via (at 117.2 62.6) (size 0.7) (drill 0.3) (layers "F.Cu" "B.Cu") (free yes) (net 1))
 (via (at 104.9 62.7) (size 0.7) (drill 0.3) (layers "F.Cu" "B.Cu") (free yes) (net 1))
 (via (at 111.9 62.6) (size 0.7) (drill 0.3) (layers "F.Cu" "B.Cu") (free yes) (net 1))
 (via (at 94.25 59.5) (size 0.7) (drill 0.3) (layers "F.Cu" "B.Cu") (free yes) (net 1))
 (via (at 97.25 59.5) (size 0.7) (drill 0.3) (layers "F.Cu" "B.Cu") (free yes) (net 1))
 (via (at 97.25 62.75) (size 0.7) (drill 0.3) (layers "F.Cu" "B.Cu") (free yes) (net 1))
 (via (at 95.75 59.5) (size 0.7) (drill 0.3) (layers "F.Cu" "B.Cu") (free yes) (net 1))
 (via (at 97.25 61) (size 0.7) (drill 0.3) (layers "F.Cu" "B.Cu") (free yes) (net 1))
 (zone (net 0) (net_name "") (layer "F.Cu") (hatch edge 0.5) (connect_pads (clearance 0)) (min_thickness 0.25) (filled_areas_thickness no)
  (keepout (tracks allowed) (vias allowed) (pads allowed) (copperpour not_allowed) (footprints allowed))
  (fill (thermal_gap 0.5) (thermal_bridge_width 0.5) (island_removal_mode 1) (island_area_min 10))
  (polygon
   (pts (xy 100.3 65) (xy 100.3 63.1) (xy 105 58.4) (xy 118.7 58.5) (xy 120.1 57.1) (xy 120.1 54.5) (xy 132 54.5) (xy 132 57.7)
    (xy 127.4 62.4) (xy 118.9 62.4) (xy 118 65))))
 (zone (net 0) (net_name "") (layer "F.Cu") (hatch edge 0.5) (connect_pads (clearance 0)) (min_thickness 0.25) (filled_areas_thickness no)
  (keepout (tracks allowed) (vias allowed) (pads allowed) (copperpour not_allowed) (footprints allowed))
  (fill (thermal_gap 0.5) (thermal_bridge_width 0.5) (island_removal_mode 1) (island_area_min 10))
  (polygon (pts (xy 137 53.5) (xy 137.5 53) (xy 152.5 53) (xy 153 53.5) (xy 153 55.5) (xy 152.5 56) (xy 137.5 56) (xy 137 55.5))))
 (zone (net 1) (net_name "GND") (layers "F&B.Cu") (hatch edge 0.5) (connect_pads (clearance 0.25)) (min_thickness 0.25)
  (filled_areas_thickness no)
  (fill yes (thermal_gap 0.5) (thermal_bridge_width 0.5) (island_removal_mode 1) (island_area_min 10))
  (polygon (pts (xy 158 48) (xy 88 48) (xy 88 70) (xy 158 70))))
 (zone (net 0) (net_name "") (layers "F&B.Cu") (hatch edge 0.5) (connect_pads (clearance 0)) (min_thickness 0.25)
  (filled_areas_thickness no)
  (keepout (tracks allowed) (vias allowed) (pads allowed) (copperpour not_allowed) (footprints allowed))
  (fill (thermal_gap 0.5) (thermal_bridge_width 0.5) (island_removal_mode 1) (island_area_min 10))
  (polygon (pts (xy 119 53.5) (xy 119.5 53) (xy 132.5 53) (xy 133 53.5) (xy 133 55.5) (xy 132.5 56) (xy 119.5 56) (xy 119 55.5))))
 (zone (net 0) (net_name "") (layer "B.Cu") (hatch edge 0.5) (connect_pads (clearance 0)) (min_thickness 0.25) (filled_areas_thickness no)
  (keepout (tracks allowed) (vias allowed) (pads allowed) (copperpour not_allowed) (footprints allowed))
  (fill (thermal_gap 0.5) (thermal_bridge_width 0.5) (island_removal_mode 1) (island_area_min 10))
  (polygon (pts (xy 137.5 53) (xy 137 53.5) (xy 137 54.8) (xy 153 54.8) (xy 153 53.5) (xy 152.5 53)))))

